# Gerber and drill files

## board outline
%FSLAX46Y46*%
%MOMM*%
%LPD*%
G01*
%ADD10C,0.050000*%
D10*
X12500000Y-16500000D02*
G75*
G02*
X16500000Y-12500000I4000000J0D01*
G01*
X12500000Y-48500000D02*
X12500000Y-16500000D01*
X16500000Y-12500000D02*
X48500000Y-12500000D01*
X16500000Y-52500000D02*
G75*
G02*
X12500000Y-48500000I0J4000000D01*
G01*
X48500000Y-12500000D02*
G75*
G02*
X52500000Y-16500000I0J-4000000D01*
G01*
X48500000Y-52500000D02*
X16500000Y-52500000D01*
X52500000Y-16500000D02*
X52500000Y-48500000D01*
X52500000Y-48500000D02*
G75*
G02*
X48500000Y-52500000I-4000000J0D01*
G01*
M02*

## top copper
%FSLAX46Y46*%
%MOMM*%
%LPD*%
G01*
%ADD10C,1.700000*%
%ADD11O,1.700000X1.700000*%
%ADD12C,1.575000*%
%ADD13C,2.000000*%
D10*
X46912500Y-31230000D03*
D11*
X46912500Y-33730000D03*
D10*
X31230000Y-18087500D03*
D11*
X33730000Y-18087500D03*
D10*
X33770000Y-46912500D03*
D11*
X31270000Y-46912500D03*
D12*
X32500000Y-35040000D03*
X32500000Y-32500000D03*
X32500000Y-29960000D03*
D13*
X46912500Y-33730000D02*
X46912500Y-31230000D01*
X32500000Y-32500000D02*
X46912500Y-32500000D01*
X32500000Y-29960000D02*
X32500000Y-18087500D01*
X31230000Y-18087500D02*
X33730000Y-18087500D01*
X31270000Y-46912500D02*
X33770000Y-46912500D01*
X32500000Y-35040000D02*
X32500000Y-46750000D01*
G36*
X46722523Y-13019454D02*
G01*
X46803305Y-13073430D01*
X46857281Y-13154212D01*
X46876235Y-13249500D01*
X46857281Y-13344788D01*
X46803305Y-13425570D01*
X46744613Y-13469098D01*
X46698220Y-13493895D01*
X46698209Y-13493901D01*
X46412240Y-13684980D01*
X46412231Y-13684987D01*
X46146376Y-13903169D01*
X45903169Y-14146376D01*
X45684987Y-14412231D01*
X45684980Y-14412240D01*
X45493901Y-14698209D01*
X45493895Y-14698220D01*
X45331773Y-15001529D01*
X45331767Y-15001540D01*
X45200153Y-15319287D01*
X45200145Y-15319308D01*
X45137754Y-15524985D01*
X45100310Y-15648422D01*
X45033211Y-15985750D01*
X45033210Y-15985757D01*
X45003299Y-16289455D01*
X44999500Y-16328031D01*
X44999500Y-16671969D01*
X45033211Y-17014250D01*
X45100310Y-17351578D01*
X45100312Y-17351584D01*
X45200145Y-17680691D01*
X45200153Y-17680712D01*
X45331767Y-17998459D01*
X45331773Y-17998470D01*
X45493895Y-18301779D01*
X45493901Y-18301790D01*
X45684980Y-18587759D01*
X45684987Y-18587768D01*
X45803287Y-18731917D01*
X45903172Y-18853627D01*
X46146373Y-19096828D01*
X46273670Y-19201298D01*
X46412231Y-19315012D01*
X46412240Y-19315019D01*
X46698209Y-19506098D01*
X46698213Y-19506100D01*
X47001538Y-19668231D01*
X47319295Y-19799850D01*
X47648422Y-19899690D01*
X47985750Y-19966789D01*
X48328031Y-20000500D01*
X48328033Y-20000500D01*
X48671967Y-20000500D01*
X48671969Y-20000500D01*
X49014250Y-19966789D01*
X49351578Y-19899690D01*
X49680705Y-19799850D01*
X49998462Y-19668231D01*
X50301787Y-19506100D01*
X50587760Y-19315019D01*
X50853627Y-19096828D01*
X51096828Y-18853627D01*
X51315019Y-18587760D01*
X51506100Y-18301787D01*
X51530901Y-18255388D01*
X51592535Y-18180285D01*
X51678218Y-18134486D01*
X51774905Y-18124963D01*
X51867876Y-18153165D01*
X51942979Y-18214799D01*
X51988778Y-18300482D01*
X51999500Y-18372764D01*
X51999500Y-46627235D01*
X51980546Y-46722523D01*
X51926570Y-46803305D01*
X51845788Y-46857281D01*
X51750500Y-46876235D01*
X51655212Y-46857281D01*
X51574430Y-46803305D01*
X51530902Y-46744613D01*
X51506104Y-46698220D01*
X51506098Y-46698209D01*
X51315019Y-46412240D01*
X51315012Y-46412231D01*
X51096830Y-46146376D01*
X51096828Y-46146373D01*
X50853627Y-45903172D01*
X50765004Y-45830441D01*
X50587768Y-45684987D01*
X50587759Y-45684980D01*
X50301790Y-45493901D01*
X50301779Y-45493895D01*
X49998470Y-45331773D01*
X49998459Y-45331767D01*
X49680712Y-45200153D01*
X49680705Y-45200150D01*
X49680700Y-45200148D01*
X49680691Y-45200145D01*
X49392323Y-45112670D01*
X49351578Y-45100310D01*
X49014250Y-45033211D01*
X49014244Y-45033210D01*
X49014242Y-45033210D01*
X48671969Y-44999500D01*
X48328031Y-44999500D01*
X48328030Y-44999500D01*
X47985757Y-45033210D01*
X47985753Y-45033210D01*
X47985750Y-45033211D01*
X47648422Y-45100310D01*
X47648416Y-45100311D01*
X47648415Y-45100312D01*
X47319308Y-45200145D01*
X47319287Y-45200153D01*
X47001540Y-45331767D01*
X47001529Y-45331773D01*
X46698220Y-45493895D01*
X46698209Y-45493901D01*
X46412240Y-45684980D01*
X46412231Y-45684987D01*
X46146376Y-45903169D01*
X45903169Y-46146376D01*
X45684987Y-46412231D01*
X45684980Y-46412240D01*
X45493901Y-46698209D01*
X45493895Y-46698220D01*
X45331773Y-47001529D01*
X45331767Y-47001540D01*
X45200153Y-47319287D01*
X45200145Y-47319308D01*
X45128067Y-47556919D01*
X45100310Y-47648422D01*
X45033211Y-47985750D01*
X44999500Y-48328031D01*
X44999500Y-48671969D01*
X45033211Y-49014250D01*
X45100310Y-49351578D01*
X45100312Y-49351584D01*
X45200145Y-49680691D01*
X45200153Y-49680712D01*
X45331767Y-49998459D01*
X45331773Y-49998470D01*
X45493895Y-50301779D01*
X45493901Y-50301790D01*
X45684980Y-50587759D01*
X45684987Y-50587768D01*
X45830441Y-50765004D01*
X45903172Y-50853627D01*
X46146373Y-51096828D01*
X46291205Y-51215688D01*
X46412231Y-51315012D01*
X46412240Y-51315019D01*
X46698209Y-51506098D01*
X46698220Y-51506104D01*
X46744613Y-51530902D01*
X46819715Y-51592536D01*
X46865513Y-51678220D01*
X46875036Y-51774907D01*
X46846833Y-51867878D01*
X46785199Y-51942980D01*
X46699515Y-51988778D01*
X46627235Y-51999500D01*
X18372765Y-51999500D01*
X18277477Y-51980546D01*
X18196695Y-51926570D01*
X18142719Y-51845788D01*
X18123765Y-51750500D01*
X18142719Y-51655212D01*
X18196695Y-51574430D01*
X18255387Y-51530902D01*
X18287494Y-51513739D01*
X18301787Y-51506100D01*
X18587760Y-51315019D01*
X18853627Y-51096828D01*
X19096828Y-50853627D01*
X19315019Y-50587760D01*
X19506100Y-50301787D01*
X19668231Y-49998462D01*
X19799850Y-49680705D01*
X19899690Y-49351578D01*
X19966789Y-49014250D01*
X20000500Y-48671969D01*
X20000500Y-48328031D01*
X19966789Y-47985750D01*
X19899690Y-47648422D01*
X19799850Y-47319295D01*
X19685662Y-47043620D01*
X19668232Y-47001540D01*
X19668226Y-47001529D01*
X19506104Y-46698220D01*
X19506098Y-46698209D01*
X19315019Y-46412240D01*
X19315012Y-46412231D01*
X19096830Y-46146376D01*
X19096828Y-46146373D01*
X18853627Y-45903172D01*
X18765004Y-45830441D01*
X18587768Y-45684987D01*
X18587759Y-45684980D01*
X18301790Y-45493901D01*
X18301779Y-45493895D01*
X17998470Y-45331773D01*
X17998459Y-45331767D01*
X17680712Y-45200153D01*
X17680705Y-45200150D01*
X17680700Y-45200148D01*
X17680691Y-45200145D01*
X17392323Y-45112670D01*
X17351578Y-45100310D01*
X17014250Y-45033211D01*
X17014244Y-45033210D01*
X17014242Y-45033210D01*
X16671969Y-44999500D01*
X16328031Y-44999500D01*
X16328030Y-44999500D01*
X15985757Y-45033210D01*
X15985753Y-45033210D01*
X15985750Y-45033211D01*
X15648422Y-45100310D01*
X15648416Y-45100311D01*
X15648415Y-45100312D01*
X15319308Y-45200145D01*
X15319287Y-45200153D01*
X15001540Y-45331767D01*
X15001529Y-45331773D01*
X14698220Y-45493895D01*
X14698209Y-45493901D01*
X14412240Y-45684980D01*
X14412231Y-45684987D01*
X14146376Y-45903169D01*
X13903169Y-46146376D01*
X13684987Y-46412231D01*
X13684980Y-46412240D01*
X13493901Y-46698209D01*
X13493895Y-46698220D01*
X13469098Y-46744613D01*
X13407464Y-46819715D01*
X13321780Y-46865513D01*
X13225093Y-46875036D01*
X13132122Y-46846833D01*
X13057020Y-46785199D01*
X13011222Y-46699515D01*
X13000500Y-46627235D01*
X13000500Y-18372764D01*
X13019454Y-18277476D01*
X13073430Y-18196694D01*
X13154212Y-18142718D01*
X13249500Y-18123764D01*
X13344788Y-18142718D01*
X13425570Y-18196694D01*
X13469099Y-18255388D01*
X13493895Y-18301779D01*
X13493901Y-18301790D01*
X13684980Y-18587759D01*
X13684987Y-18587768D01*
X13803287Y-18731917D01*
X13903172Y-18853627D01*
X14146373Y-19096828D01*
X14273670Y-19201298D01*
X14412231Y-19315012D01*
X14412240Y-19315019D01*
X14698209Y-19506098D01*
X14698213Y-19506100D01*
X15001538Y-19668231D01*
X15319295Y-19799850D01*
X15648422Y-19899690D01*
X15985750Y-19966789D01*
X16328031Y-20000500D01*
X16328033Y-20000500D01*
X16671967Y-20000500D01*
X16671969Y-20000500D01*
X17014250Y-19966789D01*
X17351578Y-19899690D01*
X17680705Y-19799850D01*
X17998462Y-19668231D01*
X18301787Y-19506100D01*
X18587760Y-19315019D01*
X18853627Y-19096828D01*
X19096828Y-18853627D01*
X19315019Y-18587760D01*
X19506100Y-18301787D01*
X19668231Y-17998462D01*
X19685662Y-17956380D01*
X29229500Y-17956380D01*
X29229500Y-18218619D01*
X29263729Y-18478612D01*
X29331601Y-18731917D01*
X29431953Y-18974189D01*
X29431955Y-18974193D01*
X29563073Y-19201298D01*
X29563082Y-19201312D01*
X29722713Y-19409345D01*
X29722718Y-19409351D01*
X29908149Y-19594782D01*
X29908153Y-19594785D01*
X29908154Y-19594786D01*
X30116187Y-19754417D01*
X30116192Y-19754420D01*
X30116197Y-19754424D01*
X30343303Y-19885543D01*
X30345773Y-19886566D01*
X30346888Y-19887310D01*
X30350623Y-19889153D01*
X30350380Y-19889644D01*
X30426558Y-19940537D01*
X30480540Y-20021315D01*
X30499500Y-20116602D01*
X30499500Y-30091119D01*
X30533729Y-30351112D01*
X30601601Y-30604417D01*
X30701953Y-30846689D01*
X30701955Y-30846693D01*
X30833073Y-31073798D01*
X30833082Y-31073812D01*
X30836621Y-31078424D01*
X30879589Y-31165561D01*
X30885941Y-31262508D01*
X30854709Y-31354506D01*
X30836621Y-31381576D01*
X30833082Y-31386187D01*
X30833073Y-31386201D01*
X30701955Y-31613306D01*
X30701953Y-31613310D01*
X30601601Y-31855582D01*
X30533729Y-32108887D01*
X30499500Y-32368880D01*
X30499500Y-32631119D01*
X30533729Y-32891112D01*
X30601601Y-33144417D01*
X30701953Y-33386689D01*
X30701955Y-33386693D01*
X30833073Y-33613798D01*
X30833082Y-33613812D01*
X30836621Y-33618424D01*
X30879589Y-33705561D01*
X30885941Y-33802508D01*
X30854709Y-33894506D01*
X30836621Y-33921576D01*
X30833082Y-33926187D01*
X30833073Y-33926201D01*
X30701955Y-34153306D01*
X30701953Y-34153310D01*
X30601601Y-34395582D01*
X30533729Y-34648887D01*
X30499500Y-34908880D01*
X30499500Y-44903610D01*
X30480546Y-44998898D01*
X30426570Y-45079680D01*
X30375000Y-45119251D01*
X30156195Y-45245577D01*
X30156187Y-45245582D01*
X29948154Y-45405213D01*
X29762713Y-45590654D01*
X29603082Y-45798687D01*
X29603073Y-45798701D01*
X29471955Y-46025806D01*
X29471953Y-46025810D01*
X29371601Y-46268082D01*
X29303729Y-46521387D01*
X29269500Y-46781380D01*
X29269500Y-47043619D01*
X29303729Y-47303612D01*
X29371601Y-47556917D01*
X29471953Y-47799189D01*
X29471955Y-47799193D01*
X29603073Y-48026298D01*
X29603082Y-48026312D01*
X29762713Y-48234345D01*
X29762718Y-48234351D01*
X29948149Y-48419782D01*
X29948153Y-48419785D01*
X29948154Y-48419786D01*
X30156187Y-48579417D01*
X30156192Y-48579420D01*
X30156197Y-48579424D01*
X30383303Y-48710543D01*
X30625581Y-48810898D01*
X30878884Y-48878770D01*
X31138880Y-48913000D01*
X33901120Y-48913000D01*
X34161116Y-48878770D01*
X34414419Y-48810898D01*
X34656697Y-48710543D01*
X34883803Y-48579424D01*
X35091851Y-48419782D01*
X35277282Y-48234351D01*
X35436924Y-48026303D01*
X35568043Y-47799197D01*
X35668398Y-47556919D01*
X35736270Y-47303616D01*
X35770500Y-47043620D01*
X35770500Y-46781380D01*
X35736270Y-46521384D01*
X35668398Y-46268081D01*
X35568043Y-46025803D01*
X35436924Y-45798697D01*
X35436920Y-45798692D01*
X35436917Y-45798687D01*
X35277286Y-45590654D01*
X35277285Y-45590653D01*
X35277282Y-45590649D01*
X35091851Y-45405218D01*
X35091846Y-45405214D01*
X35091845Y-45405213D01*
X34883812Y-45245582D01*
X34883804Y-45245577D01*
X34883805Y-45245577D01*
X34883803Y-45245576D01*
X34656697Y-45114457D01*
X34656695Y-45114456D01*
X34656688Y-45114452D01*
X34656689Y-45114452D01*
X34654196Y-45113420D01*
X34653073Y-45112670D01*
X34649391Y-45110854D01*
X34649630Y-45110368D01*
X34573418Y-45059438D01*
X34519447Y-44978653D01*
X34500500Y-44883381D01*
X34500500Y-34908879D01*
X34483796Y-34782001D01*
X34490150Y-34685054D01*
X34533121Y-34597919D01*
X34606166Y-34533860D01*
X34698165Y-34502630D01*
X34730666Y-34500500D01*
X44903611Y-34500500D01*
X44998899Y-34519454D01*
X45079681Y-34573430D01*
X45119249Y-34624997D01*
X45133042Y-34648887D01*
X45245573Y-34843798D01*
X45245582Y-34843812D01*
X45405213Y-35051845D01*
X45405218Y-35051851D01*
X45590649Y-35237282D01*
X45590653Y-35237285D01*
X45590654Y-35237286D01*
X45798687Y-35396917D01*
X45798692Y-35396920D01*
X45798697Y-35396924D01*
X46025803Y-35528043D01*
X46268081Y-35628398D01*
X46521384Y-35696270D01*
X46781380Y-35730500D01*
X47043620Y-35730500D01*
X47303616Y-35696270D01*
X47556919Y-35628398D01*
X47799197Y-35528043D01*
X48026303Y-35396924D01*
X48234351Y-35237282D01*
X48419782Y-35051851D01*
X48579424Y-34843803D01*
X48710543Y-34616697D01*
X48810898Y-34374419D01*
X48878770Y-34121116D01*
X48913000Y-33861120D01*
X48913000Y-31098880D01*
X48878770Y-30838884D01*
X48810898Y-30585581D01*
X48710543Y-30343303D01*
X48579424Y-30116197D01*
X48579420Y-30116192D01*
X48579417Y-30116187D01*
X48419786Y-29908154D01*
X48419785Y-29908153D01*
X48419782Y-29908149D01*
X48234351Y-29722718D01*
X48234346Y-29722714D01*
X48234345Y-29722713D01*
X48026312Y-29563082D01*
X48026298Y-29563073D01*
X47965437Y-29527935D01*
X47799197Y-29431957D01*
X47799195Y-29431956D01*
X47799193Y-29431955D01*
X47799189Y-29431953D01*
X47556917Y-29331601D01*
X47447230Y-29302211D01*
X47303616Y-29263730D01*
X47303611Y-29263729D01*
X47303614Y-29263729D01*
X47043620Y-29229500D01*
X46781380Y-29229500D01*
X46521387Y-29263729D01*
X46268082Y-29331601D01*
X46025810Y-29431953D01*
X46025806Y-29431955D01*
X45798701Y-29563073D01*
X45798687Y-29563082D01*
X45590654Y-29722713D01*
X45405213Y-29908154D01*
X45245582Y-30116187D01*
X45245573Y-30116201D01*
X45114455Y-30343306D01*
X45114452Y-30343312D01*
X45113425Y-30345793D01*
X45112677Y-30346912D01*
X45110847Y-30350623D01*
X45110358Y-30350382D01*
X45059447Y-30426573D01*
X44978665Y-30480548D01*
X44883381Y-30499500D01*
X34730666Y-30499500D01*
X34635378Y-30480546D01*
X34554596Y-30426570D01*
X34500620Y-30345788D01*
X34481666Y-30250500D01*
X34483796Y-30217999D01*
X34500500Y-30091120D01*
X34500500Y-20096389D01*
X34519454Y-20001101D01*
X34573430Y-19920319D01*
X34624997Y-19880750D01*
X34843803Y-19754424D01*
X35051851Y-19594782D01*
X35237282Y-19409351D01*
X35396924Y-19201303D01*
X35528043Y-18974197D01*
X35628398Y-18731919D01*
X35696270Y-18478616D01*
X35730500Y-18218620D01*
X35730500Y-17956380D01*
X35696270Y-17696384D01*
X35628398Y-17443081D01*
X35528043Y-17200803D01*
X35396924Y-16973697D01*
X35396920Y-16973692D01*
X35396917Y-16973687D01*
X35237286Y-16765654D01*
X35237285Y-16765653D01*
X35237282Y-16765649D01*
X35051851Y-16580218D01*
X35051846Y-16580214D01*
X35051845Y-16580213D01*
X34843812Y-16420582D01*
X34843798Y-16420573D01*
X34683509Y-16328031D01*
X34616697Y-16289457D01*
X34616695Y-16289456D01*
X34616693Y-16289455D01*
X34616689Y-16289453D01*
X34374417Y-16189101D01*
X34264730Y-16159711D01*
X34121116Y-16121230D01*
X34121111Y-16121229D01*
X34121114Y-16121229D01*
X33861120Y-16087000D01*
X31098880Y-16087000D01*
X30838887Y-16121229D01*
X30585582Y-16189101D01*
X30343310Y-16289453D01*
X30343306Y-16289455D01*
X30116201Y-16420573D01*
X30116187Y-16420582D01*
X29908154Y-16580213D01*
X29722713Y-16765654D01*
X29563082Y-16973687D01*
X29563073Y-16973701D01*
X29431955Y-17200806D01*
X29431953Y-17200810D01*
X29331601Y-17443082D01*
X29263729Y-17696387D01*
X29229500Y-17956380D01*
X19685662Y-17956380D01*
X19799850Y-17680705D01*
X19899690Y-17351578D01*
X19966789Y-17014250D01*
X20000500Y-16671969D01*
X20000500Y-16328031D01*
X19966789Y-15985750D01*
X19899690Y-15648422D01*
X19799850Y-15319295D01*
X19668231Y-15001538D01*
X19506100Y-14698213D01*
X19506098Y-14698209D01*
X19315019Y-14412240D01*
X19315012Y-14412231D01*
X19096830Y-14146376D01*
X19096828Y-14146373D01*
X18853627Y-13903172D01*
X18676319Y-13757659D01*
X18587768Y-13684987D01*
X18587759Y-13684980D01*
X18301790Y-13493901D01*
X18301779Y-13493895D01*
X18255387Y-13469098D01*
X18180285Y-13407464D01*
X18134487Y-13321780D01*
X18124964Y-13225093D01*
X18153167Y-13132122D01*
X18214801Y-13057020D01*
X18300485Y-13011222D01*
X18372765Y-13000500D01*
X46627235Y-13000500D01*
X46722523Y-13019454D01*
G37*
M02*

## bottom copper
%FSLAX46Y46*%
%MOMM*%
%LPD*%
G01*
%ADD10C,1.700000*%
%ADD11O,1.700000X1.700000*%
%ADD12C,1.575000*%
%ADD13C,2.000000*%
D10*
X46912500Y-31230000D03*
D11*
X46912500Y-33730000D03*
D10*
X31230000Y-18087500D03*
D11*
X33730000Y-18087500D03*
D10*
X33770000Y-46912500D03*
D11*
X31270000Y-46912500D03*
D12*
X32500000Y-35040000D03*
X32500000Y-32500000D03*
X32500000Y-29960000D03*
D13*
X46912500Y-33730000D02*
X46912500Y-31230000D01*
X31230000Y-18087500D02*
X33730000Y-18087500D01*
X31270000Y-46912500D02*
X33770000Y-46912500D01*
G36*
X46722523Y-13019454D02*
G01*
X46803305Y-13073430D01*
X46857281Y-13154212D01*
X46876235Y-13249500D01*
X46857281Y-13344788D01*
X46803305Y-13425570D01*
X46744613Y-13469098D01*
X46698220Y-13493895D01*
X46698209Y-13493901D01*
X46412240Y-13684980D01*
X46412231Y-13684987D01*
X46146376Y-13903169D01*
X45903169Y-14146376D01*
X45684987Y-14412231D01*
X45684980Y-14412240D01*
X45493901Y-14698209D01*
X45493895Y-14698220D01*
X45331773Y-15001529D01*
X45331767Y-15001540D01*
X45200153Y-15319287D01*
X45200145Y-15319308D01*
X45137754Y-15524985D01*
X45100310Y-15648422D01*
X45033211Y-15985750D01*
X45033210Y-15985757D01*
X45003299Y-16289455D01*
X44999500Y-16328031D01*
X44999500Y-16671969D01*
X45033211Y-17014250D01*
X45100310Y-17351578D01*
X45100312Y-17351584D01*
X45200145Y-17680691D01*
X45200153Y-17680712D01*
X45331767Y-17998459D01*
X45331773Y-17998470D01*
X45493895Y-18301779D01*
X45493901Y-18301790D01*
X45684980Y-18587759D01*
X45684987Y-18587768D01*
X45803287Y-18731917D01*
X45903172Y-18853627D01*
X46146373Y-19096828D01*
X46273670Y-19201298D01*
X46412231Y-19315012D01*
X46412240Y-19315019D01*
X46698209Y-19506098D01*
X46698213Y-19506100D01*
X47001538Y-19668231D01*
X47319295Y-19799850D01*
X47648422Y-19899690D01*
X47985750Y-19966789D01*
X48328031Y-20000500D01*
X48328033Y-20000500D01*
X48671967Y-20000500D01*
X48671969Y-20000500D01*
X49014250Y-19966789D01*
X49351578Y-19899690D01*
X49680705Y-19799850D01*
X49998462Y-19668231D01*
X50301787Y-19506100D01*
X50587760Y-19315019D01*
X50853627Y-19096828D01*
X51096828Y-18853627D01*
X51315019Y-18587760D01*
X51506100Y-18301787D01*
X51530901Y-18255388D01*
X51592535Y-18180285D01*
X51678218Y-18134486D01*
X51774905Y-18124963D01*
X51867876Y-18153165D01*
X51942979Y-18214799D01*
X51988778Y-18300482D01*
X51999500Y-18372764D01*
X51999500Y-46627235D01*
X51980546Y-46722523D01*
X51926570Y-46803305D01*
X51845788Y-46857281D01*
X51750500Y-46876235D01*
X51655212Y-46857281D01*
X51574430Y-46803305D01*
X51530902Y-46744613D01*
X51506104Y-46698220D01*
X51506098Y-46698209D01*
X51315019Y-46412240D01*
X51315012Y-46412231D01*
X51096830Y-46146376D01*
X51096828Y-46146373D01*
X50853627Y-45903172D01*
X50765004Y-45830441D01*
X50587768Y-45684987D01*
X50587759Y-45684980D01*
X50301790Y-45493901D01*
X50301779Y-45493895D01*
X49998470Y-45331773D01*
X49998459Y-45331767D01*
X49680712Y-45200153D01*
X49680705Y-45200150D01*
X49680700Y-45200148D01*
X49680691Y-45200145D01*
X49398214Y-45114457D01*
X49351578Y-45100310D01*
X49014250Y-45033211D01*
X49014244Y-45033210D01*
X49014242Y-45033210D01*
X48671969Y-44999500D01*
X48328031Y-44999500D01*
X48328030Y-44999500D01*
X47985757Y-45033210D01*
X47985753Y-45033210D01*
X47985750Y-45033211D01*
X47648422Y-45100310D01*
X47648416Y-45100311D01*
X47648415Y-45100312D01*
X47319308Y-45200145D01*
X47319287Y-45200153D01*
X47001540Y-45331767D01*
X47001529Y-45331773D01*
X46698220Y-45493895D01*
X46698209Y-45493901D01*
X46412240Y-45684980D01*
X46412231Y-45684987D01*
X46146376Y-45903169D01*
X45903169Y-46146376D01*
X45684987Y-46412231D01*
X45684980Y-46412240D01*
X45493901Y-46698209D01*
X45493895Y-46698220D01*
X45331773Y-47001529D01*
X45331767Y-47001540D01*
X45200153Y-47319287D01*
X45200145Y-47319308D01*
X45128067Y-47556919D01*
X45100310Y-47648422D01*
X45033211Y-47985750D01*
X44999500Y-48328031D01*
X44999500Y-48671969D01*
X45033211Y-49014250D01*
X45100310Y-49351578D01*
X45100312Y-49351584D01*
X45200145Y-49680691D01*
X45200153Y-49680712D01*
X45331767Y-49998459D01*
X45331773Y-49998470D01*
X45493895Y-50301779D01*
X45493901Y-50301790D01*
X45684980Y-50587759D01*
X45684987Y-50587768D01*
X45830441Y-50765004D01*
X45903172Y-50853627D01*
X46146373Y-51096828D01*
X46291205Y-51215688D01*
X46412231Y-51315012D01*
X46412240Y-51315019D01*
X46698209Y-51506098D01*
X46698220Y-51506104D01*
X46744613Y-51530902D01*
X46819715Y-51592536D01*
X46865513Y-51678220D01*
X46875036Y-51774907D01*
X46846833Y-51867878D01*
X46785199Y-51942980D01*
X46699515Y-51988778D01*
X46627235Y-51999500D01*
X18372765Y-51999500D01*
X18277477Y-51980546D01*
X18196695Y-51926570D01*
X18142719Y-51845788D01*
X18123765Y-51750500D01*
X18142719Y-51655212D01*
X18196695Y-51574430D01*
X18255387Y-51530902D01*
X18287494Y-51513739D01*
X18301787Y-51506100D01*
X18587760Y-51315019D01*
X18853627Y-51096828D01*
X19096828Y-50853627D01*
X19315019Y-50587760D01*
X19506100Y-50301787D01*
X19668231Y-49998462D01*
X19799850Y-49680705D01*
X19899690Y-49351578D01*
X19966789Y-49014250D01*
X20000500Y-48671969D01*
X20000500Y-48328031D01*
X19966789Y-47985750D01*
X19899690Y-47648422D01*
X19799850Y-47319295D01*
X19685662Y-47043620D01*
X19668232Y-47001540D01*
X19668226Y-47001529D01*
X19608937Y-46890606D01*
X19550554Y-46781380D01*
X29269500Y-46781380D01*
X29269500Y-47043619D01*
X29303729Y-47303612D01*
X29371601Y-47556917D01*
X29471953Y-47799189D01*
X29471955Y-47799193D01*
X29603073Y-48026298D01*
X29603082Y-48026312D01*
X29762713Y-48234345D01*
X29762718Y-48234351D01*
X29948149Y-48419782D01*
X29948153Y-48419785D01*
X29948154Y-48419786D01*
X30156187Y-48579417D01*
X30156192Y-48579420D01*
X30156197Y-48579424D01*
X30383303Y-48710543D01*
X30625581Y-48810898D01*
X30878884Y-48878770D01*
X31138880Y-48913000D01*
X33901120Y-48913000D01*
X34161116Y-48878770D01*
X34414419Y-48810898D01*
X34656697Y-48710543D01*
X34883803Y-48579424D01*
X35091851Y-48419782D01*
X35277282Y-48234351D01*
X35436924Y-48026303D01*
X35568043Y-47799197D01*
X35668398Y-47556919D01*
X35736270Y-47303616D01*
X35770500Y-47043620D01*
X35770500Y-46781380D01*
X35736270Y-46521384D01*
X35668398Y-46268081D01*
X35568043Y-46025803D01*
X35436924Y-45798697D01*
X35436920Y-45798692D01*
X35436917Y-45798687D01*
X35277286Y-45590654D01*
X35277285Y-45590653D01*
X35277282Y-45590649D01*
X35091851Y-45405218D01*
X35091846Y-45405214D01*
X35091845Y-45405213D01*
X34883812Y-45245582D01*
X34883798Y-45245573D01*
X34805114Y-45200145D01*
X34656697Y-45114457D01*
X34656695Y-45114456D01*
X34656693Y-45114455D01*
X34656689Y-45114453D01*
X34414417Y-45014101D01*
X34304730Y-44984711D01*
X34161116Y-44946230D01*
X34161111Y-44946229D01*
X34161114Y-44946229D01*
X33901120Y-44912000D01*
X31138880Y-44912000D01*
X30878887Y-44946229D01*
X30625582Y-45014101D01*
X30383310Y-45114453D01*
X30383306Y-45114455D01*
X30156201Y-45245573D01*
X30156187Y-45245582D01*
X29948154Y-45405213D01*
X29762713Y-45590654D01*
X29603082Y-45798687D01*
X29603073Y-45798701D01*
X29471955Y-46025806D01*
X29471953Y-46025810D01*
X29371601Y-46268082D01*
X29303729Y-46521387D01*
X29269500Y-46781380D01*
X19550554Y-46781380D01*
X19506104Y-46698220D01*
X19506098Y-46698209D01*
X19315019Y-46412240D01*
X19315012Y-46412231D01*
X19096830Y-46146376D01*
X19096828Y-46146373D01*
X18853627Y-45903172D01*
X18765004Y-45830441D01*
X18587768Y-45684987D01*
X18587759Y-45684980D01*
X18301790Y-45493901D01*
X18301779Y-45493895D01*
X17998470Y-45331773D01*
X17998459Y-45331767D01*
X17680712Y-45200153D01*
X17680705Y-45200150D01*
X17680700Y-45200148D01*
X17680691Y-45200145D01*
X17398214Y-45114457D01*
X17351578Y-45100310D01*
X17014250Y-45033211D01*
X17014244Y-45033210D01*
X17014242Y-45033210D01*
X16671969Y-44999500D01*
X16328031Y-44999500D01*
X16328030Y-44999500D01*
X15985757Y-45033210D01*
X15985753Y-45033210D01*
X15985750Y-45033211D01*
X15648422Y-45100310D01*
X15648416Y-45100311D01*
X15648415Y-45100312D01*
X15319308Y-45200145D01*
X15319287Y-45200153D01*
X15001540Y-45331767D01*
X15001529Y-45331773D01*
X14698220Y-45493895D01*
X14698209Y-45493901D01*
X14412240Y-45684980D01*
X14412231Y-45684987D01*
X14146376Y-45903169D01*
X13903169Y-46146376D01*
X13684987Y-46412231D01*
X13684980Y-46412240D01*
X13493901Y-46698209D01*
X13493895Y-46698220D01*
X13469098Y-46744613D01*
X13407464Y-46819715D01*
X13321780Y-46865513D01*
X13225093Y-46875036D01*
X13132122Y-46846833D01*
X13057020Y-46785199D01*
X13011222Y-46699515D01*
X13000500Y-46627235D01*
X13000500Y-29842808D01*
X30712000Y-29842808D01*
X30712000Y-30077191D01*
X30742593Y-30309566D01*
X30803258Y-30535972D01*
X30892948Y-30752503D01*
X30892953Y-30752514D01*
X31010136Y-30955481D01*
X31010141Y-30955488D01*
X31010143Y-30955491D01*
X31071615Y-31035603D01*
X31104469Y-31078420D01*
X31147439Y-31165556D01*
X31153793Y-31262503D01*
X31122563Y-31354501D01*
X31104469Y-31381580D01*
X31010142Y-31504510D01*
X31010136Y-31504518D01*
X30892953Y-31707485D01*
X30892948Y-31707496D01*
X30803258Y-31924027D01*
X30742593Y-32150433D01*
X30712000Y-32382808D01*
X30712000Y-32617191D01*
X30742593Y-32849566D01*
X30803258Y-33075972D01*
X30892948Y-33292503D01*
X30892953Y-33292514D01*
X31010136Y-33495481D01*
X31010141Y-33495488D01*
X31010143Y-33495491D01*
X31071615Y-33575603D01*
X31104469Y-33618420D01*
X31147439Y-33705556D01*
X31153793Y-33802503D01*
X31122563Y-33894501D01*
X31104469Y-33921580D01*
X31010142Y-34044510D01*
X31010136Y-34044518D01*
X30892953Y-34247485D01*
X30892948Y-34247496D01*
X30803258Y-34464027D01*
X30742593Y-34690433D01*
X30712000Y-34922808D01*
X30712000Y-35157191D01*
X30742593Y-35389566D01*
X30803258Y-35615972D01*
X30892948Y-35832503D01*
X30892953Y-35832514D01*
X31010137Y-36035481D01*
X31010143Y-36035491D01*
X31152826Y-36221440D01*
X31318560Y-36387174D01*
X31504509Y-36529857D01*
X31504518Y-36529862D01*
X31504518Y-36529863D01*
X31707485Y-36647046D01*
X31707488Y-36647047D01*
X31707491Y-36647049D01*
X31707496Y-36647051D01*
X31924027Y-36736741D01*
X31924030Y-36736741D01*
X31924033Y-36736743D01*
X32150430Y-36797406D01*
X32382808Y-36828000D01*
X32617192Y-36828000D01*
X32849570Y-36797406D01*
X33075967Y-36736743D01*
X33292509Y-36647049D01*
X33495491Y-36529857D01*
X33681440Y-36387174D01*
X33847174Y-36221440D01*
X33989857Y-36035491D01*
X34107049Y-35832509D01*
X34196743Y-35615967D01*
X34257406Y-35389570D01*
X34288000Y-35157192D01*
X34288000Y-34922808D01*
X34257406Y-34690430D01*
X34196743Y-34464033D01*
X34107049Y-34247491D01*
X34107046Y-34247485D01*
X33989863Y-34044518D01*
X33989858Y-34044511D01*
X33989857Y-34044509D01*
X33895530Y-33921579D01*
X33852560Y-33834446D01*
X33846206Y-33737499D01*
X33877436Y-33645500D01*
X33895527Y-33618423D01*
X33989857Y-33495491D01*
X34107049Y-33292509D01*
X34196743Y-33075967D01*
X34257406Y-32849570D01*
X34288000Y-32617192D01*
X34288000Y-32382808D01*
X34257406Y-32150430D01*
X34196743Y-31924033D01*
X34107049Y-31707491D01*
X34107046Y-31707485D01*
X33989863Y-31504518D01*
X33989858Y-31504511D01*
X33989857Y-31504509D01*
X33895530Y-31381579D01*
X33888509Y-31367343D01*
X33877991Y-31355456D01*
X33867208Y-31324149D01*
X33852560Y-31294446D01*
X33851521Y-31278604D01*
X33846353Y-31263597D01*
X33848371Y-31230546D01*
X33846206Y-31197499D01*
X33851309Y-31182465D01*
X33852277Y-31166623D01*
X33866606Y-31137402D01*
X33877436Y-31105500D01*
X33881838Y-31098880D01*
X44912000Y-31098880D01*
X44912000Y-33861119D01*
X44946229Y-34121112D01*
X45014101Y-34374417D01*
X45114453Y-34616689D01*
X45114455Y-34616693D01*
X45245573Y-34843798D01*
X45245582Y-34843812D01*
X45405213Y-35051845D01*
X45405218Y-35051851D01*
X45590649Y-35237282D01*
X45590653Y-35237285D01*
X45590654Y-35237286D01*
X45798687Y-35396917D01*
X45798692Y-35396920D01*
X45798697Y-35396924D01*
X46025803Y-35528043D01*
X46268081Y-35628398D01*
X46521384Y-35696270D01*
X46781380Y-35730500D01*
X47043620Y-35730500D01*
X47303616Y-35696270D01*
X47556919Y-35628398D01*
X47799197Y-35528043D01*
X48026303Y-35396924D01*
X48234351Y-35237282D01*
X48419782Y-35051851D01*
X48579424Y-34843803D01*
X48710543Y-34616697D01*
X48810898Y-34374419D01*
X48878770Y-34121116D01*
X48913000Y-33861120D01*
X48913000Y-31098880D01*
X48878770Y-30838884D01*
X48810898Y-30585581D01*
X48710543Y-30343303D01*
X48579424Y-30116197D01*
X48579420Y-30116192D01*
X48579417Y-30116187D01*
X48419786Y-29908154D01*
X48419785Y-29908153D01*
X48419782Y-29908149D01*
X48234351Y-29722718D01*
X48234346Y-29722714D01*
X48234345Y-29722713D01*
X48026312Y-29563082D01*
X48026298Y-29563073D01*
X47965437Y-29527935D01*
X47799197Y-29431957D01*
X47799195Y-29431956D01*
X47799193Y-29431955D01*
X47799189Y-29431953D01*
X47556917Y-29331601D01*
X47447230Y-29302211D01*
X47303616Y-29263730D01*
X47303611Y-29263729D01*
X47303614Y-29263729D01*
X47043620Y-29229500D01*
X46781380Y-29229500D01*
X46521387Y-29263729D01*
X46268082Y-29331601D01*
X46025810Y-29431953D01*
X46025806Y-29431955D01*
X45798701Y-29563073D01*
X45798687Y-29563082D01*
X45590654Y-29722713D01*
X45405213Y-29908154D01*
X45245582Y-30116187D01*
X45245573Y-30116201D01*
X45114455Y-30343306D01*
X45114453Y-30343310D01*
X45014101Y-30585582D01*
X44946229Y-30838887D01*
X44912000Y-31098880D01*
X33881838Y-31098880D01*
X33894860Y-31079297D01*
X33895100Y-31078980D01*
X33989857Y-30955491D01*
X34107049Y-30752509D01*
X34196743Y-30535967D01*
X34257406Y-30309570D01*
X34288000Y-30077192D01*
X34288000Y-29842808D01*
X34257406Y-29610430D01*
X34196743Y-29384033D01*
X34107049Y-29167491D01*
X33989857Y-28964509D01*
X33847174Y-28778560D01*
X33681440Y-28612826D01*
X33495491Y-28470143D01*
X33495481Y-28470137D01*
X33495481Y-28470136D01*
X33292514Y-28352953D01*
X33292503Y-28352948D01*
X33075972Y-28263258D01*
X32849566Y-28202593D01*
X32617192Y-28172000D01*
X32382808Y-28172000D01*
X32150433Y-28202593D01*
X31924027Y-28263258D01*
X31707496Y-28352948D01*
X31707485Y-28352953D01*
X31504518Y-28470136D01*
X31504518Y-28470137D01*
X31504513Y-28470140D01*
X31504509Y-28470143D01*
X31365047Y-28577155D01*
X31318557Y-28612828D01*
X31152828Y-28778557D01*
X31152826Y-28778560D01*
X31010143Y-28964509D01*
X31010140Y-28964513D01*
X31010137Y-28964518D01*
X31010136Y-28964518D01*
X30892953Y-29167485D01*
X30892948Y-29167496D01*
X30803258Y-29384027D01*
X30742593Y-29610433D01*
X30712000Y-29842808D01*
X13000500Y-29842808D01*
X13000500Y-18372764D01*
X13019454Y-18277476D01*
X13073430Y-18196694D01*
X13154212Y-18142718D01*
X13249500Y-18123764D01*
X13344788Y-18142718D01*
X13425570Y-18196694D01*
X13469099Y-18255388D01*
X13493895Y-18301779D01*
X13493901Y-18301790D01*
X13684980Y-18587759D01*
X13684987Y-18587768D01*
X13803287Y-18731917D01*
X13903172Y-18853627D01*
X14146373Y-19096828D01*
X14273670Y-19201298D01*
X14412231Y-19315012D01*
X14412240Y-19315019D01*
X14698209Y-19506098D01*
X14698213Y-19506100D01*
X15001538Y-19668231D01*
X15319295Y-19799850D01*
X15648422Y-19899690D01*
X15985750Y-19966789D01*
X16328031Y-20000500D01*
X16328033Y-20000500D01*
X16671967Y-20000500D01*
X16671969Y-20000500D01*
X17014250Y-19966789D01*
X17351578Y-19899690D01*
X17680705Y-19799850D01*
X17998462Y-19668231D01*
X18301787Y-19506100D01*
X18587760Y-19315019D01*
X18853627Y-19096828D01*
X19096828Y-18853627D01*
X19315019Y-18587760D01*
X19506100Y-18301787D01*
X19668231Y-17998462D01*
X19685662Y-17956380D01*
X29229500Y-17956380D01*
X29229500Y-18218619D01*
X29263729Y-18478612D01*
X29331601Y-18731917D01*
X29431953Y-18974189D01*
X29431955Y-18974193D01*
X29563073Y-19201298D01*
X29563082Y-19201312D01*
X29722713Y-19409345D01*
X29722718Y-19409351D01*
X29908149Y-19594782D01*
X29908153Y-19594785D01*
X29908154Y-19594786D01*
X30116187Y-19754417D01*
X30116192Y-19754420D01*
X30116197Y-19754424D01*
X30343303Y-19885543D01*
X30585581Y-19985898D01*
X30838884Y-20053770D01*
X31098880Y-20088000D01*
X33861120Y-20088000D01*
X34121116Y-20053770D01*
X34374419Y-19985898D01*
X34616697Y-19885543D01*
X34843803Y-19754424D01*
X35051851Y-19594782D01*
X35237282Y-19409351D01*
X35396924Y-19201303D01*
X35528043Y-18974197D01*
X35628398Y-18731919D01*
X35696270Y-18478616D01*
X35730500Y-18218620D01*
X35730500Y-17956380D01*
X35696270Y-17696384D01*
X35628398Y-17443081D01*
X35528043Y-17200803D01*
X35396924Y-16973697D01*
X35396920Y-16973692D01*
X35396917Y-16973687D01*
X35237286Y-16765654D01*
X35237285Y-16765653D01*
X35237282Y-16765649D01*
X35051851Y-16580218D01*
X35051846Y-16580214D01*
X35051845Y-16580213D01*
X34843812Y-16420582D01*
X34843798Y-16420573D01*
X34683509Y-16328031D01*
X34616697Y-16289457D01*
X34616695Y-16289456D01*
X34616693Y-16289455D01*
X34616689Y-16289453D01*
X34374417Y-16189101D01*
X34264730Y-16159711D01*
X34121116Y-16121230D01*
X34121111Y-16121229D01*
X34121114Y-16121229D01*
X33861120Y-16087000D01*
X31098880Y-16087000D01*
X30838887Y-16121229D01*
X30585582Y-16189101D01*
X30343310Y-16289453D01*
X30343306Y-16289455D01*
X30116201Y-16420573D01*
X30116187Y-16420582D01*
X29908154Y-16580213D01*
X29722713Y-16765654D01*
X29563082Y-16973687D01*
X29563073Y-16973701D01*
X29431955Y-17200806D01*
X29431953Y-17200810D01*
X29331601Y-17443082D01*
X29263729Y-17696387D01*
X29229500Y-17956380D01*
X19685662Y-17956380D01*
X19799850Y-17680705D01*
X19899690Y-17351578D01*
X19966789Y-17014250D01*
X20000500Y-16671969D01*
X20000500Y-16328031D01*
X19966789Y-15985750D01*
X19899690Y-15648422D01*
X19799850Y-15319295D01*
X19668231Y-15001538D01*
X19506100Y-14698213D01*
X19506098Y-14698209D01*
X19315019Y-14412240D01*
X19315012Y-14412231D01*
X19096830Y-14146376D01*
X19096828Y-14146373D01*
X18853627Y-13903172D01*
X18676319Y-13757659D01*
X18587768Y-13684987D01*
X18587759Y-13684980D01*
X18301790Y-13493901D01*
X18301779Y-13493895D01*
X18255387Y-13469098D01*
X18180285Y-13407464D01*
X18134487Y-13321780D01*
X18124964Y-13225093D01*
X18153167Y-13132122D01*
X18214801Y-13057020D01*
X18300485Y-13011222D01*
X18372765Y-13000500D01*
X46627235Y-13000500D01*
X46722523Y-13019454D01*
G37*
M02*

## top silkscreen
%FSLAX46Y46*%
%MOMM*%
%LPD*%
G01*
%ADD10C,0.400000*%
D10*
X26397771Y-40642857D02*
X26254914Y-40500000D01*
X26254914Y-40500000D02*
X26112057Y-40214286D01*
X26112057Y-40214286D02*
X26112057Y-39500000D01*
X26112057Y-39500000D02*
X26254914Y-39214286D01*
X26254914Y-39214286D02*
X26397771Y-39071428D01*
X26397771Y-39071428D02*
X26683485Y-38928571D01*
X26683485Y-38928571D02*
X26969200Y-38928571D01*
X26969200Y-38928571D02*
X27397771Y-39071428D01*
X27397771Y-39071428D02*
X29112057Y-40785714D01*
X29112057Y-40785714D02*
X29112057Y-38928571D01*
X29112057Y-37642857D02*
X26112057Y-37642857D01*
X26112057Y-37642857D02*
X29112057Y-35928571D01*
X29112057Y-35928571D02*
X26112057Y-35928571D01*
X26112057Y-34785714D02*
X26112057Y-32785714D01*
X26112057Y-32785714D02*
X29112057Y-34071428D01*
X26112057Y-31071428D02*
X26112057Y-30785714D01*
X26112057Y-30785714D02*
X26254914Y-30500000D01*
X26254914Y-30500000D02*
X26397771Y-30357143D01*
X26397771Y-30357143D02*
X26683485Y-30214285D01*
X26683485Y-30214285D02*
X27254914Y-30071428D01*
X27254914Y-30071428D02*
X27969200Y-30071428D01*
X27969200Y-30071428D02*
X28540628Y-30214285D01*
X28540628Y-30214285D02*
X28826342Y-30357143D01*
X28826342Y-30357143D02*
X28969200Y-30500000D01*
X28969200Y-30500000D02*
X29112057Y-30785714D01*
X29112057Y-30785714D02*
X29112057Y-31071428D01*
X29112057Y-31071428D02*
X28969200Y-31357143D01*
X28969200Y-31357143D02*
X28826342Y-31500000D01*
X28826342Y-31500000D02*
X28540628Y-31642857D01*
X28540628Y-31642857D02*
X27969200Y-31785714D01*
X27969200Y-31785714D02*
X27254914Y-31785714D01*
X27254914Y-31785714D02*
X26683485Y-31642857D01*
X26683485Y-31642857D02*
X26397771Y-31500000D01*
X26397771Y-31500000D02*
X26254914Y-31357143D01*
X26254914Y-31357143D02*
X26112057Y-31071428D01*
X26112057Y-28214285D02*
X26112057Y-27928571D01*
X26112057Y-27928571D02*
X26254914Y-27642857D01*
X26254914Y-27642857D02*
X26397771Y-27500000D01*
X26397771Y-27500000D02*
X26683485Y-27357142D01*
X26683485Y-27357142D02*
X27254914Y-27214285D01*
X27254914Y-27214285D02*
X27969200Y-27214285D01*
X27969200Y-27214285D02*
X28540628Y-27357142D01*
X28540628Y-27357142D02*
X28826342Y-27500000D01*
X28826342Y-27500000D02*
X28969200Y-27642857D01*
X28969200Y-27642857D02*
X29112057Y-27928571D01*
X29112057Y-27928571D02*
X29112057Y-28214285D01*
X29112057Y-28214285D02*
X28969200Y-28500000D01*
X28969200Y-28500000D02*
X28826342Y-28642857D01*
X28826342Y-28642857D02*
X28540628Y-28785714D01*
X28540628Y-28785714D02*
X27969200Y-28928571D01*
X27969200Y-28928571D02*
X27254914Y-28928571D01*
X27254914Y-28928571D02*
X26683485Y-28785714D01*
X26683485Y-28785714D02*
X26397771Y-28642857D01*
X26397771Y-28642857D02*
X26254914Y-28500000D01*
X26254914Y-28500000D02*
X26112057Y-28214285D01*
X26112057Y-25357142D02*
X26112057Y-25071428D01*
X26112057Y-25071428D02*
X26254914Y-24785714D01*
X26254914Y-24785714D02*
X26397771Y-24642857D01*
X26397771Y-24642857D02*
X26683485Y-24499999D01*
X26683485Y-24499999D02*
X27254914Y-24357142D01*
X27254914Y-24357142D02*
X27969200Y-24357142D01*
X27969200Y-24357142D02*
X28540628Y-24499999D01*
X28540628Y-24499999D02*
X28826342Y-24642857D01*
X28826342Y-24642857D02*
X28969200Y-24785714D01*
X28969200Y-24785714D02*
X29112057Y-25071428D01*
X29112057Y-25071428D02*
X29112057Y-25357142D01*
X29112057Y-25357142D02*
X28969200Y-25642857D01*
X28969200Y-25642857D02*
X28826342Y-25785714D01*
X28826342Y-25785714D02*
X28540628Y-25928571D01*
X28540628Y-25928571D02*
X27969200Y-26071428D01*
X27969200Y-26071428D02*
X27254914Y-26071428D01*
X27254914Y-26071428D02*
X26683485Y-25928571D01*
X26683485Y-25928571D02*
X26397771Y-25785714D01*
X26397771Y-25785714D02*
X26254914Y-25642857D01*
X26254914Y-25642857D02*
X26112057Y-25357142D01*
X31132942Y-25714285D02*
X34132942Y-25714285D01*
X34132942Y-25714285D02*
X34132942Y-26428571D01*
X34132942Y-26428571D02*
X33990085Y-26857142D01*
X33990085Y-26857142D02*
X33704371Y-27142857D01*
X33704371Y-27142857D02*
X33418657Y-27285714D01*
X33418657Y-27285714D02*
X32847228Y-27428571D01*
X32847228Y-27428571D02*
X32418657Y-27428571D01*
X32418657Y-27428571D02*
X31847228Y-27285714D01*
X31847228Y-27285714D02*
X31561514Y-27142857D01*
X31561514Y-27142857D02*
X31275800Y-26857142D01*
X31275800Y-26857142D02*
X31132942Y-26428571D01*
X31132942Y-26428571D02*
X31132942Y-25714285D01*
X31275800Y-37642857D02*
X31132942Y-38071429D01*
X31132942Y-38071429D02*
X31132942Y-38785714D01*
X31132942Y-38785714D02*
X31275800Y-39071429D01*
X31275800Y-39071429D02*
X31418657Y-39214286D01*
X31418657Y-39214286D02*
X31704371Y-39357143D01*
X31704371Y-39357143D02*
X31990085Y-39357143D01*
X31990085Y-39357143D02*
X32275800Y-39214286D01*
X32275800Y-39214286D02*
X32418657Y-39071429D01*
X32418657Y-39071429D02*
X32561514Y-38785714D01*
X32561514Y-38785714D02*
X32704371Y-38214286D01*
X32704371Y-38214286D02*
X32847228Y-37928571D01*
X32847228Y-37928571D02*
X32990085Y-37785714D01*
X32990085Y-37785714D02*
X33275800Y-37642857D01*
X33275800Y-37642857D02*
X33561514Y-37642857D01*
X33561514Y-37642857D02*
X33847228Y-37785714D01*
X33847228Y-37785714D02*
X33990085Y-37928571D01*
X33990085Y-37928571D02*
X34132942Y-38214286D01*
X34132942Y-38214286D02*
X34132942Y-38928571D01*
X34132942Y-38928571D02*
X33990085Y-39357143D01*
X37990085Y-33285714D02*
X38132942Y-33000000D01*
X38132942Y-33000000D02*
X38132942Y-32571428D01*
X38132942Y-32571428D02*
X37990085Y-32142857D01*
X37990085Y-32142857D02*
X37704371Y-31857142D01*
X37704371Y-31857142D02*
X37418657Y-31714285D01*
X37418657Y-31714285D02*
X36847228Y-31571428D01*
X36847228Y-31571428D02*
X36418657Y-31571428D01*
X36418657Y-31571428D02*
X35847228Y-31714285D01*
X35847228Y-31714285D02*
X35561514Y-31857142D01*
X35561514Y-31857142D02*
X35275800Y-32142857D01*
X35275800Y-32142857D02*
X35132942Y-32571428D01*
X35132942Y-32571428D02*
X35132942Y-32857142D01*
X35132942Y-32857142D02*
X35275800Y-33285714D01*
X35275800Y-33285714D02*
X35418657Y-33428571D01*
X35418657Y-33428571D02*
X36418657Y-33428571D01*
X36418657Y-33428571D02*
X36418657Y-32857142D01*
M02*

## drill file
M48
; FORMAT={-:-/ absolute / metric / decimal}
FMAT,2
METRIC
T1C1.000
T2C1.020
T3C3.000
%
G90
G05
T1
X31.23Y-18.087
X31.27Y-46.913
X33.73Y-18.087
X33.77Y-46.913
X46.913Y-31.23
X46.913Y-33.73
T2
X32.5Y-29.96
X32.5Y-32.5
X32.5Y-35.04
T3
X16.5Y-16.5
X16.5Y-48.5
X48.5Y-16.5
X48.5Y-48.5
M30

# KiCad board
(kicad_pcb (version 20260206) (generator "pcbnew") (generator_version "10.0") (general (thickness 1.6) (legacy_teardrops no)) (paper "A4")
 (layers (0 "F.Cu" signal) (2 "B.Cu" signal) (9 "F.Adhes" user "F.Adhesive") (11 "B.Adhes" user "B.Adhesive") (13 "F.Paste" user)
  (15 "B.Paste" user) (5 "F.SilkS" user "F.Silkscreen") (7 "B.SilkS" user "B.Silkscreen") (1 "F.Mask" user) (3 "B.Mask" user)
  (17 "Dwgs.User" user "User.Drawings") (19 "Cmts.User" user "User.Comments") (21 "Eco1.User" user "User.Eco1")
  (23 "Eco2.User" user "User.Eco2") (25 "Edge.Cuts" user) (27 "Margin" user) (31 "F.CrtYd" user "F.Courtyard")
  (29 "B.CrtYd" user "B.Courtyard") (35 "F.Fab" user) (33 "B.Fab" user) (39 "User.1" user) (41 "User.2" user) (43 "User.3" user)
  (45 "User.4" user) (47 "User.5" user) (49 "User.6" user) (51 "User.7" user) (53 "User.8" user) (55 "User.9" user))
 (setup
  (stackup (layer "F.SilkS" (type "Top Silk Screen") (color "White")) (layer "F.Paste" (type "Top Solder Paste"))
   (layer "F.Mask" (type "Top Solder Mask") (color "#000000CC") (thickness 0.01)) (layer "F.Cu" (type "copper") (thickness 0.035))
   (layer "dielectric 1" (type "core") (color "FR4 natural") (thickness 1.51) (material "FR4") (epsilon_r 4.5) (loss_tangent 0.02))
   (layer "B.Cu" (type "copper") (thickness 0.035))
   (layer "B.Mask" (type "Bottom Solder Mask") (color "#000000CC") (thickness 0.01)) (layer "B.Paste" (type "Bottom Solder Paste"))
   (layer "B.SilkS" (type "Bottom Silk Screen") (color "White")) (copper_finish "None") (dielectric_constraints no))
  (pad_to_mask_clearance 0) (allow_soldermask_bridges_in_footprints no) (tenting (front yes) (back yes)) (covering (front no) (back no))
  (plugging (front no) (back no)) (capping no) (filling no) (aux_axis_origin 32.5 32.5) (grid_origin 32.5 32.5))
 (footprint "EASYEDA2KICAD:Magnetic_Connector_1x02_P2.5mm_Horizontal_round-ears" (layer "F.Cu") (at 47.0125 32.5)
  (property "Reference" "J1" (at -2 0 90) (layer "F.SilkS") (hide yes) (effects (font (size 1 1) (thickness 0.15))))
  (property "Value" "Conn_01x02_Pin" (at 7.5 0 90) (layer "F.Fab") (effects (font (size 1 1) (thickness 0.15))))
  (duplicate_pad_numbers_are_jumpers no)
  (pad "1" thru_hole circle (at -0.1 -1.27) (size 1.7 1.7) (drill 1) (layers "*.Cu" "*.Mask") (remove_unused_layers no)
   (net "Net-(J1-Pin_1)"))
  (pad "2" thru_hole oval (at -0.1 1.23) (size 1.7 1.7) (drill 1) (layers "*.Cu" "*.Mask") (remove_unused_layers no) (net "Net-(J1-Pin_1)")))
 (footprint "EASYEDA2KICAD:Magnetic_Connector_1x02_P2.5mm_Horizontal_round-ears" (layer "F.Cu") (at 32.5 17.9875 90)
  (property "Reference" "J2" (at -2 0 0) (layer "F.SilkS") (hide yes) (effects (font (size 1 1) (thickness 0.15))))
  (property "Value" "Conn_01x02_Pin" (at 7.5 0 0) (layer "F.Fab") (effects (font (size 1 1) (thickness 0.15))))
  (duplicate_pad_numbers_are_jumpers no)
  (pad "1" thru_hole circle (at -0.1 -1.27 90) (size 1.7 1.7) (drill 1) (layers "*.Cu" "*.Mask") (remove_unused_layers no)
   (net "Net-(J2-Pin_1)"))
  (pad "2" thru_hole oval (at -0.1 1.23 90) (size 1.7 1.7) (drill 1) (layers "*.Cu" "*.Mask") (remove_unused_layers no)
   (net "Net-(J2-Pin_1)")))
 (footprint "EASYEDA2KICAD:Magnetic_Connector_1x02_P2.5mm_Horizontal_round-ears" (layer "F.Cu") (at 32.5 47.0125 -90)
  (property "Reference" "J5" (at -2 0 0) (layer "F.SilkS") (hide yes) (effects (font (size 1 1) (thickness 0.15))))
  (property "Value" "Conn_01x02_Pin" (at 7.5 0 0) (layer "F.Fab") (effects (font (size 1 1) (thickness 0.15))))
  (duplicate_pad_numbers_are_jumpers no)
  (pad "1" thru_hole circle (at -0.1 -1.27 270) (size 1.7 1.7) (drill 1) (layers "*.Cu" "*.Mask") (remove_unused_layers no) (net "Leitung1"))
  (pad "2" thru_hole oval (at -0.1 1.23 270) (size 1.7 1.7) (drill 1) (layers "*.Cu" "*.Mask") (remove_unused_layers no) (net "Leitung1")))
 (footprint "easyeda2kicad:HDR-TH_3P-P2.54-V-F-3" (layer "B.Cu") (at 32.5 32.5 90)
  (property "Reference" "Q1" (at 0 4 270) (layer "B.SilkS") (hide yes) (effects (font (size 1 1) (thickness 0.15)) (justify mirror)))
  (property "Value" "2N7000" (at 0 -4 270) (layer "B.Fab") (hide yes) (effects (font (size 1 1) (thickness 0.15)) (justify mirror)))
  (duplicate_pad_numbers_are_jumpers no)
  (pad "1" thru_hole circle (at -2.54 0 90) (size 1.575 1.575) (drill 1.020014) (layers "*.Cu" "*.Mask") (remove_unused_layers no)
   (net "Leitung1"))
  (pad "2" thru_hole circle (at 0 0 90) (size 1.575 1.575) (drill 1.020014) (layers "*.Cu" "*.Mask") (remove_unused_layers no)
   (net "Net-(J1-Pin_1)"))
  (pad "3" thru_hole circle (at 2.54 0 90) (size 1.575 1.575) (drill 1.020014) (layers "*.Cu" "*.Mask") (remove_unused_layers no)
   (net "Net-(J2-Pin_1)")))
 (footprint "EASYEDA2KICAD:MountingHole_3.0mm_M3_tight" (layer "B.Cu") (at 16.5 16.5 180)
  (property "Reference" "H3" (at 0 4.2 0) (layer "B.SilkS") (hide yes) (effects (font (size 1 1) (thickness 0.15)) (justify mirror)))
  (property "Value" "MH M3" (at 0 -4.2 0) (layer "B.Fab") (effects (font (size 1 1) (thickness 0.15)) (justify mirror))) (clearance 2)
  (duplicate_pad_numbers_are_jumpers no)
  (pad "" np_thru_hole circle (at 0 0 180) (size 3 3) (drill 3) (layers "*.Cu" "*.Mask")))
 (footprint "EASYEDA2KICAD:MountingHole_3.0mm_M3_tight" (layer "B.Cu") (at 16.5 48.5 180)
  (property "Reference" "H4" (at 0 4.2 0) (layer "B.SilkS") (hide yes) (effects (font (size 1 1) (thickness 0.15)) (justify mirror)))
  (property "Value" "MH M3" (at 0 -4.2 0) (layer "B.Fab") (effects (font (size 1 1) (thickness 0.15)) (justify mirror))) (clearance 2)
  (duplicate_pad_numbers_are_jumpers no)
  (pad "" np_thru_hole circle (at 0 0 180) (size 3 3) (drill 3) (layers "*.Cu" "*.Mask")))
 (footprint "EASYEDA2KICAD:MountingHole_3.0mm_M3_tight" (layer "B.Cu") (at 48.5 16.5 180)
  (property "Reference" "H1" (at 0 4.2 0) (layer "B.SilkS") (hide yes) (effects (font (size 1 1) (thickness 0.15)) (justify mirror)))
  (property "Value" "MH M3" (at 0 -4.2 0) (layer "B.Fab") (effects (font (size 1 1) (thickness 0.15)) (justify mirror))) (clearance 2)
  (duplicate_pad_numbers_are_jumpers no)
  (pad "" np_thru_hole circle (at 0 0 180) (size 3 3) (drill 3) (layers "*.Cu" "*.Mask")))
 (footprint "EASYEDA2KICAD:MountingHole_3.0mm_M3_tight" (layer "B.Cu") (at 48.5 48.5 180)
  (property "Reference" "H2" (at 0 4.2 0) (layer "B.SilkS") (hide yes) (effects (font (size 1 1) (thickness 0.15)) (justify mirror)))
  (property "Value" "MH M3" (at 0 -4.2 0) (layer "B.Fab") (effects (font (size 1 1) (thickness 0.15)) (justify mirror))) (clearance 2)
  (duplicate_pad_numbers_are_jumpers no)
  (pad "" np_thru_hole circle (at 0 0 180) (size 3 3) (drill 3) (layers "*.Cu" "*.Mask")))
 (gr_arc (start 12.5 16.5) (mid 13.671573 13.671573) (end 16.5 12.5) (stroke (width 0.05) (type default)) (layer "Edge.Cuts"))
 (gr_line (start 12.5 48.5) (end 12.5 16.5) (stroke (width 0.05) (type default)) (layer "Edge.Cuts"))
 (gr_line (start 16.5 12.5) (end 48.5 12.5) (stroke (width 0.05) (type default)) (layer "Edge.Cuts"))
 (gr_arc (start 16.5 52.5) (mid 13.671573 51.328427) (end 12.5 48.5) (stroke (width 0.05) (type default)) (layer "Edge.Cuts"))
 (gr_arc (start 48.5 12.5) (mid 51.328427 13.671573) (end 52.5 16.5) (stroke (width 0.05) (type default)) (layer "Edge.Cuts"))
 (gr_line (start 48.5 52.5) (end 16.5 52.5) (stroke (width 0.05) (type default)) (layer "Edge.Cuts"))
 (gr_line (start 52.5 16.5) (end 52.5 48.5) (stroke (width 0.05) (type default)) (layer "Edge.Cuts"))
 (gr_arc (start 52.5 48.5) (mid 51.328427 51.328427) (end 48.5 52.5) (stroke (width 0.05) (type default)) (layer "Edge.Cuts"))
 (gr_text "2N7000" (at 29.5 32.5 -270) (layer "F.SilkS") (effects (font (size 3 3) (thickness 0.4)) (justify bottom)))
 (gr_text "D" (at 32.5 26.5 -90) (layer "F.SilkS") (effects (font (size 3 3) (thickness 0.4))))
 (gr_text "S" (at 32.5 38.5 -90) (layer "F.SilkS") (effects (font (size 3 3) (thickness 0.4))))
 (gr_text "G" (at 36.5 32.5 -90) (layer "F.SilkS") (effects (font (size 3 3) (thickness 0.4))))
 (segment (start 46.9125 33.73) (end 46.9125 31.23) (width 2) (layer "F.Cu") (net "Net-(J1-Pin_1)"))
 (segment (start 32.5 32.5) (end 46.9125 32.5) (width 2) (layer "F.Cu") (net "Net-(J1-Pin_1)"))
 (segment (start 46.9125 33.73) (end 46.9125 31.23) (width 2) (layer "B.Cu") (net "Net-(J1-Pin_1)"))
 (segment (start 32.5 29.96) (end 32.5 18.0875) (width 2) (layer "F.Cu") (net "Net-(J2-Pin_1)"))
 (segment (start 31.23 18.0875) (end 33.73 18.0875) (width 2) (layer "F.Cu") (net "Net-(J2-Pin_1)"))
 (segment (start 31.23 18.0875) (end 33.73 18.0875) (width 2) (layer "B.Cu") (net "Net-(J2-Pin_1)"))
 (segment (start 31.27 46.9125) (end 33.77 46.9125) (width 2) (layer "F.Cu") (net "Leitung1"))
 (segment (start 32.5 35.04) (end 32.5 46.75) (width 2) (layer "F.Cu") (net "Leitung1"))
 (segment (start 31.27 46.9125) (end 33.77 46.9125) (width 2) (layer "B.Cu") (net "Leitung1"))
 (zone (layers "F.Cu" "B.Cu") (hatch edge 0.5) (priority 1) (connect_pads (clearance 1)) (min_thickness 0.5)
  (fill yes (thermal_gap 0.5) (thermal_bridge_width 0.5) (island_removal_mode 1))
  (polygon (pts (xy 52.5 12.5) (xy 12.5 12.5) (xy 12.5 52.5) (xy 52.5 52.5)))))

